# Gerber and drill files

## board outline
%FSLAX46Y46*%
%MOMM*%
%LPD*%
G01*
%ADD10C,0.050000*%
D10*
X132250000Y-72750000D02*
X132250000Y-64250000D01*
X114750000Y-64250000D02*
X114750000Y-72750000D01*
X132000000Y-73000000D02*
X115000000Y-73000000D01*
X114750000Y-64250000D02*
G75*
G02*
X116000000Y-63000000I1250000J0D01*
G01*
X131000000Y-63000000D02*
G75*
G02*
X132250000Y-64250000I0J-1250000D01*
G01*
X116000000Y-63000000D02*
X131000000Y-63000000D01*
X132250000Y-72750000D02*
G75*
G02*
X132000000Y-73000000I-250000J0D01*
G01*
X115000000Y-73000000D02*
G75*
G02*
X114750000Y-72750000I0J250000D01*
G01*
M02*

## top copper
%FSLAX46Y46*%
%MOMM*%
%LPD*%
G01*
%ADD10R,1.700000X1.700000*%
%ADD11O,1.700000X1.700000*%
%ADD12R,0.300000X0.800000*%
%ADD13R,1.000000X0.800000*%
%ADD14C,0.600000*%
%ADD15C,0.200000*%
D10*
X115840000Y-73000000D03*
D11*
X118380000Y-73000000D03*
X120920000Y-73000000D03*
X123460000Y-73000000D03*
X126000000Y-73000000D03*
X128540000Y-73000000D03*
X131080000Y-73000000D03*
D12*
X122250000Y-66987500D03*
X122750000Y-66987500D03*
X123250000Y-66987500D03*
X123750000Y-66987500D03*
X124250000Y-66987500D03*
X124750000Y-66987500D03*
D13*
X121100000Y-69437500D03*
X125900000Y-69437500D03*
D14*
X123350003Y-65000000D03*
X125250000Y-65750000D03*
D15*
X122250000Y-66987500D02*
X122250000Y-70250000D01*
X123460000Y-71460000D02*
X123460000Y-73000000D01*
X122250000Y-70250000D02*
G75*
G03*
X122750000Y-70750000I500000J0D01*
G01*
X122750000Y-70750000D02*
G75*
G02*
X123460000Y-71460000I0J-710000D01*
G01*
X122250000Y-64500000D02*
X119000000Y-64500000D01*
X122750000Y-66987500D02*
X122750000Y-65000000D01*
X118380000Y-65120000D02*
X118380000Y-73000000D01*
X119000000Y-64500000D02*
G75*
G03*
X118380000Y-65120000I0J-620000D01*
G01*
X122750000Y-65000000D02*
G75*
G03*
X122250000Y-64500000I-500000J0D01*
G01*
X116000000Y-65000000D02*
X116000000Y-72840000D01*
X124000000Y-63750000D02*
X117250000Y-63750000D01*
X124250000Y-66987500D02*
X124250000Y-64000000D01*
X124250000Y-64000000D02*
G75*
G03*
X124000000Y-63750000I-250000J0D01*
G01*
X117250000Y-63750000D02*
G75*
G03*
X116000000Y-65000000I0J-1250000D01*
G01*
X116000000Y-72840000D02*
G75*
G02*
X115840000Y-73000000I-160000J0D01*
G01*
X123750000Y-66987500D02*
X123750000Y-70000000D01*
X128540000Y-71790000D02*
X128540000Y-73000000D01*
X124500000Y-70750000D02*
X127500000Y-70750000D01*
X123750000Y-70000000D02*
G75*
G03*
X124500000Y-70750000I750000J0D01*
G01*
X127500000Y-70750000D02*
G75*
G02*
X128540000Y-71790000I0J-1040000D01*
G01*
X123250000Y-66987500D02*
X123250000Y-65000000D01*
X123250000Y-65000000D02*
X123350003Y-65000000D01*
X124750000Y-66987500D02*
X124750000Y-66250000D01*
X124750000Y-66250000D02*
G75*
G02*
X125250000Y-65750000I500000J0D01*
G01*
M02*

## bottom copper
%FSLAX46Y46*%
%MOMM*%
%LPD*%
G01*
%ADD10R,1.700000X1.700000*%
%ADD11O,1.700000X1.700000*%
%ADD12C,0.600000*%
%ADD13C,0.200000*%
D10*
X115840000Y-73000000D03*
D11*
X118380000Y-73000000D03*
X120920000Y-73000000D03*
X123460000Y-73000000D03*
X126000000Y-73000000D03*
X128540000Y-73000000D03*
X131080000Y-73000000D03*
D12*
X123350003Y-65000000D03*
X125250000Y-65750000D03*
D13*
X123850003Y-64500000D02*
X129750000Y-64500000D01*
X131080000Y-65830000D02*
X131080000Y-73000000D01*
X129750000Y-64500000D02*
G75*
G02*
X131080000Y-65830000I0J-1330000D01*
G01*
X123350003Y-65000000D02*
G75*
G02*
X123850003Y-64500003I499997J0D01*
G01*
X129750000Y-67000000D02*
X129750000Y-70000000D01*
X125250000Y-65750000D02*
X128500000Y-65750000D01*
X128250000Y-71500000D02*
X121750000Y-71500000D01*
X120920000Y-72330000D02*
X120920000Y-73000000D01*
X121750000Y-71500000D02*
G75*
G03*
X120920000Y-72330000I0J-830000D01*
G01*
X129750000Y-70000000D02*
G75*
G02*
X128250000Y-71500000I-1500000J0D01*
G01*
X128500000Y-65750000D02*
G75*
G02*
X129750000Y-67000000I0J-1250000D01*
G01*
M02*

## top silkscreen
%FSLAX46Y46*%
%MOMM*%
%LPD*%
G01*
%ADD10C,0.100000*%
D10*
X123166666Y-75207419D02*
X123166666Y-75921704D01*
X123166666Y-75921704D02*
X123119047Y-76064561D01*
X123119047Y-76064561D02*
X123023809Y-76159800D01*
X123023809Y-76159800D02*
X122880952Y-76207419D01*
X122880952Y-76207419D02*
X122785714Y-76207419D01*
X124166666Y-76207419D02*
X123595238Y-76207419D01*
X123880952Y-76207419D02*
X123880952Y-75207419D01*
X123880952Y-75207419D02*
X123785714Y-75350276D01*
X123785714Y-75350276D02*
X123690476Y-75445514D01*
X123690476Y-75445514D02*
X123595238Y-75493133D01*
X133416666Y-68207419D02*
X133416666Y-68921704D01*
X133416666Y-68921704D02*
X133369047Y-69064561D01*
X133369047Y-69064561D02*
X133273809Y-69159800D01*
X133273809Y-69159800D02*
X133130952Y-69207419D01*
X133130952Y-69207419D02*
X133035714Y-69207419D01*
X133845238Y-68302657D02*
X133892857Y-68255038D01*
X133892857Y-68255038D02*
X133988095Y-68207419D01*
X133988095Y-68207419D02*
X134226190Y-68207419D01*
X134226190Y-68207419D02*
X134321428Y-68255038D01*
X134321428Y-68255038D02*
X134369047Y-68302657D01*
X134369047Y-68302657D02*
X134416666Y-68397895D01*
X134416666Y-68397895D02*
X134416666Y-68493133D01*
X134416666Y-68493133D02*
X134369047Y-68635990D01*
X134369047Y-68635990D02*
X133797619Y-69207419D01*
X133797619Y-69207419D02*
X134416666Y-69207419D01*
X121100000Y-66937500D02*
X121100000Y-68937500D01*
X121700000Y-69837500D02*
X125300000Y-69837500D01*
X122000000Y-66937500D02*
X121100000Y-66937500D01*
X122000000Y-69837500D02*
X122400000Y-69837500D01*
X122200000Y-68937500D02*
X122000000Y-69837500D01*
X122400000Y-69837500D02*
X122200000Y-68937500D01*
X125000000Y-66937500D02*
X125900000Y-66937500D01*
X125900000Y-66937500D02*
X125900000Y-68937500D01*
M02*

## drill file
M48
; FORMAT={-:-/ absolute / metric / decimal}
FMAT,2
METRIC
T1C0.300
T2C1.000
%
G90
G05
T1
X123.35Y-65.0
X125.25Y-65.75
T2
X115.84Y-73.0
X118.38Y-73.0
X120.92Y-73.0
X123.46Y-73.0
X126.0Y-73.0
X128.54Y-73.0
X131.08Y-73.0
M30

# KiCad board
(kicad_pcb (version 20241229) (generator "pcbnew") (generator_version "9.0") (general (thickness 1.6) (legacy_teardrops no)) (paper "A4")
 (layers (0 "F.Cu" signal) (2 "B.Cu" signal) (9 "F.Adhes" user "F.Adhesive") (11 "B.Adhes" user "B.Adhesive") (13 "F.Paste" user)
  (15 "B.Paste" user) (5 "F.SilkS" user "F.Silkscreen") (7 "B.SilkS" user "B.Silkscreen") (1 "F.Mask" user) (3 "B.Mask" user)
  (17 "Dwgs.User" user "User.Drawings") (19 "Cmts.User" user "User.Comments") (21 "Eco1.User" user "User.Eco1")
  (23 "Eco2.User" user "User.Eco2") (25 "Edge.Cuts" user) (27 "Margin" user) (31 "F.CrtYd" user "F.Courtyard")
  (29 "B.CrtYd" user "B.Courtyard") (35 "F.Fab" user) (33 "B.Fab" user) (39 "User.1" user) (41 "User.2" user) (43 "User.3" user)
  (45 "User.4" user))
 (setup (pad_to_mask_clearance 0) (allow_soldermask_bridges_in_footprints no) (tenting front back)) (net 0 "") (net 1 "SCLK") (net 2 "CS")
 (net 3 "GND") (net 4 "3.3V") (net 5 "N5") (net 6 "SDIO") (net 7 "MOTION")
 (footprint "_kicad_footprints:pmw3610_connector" (layer "F.Cu") (at 123.46 73 90)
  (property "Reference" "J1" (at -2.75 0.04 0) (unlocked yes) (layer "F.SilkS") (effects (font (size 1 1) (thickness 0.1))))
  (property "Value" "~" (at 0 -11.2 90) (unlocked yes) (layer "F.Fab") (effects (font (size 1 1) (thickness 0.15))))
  (pad "1" thru_hole rect (at 0 -7.62 90) (size 1.7 1.7) (drill 1) (layers "*.Cu" "*.Mask") (remove_unused_layers no) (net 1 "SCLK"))
  (pad "2" thru_hole oval (at 0 -5.08 90) (size 1.7 1.7) (drill 1) (layers "*.Cu" "*.Mask") (remove_unused_layers no) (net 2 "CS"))
  (pad "3" thru_hole oval (at 0 -2.54 90) (size 1.7 1.7) (drill 1) (layers "*.Cu" "*.Mask") (remove_unused_layers no) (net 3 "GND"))
  (pad "4" thru_hole oval (at 0 0 90) (size 1.7 1.7) (drill 1) (layers "*.Cu" "*.Mask") (remove_unused_layers no) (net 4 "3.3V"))
  (pad "5" thru_hole oval (at 0 2.54 90) (size 1.7 1.7) (drill 1) (layers "*.Cu" "*.Mask") (remove_unused_layers no) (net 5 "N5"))
  (pad "6" thru_hole oval (at 0 5.08 90) (size 1.7 1.7) (drill 1) (layers "*.Cu" "*.Mask") (remove_unused_layers no) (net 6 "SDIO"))
  (pad "7" thru_hole oval (at 0 7.62 90) (size 1.7 1.7) (drill 1) (layers "*.Cu" "*.Mask") (remove_unused_layers no) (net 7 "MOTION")))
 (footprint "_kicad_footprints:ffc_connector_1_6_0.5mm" (layer "F.Cu") (at 123.5 75.2375)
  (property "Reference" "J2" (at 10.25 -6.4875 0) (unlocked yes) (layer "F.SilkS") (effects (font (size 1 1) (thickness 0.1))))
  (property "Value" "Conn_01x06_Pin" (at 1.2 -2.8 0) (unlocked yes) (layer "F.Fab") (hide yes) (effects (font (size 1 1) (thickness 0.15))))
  (fp_line (start -2.4 -8.3) (end -2.4 -6.3) (stroke (width 0.1) (type default)) (layer "F.SilkS"))
  (fp_line (start -1.8 -5.4) (end 1.8 -5.4) (stroke (width 0.1) (type default)) (layer "F.SilkS"))
  (fp_line (start -1.5 -8.3) (end -2.4 -8.3) (stroke (width 0.1) (type default)) (layer "F.SilkS"))
  (fp_line (start -1.5 -5.4) (end -1.1 -5.4) (stroke (width 0.1) (type default)) (layer "F.SilkS"))
  (fp_line (start -1.3 -6.3) (end -1.5 -5.4) (stroke (width 0.1) (type default)) (layer "F.SilkS"))
  (fp_line (start -1.1 -5.4) (end -1.3 -6.3) (stroke (width 0.1) (type default)) (layer "F.SilkS"))
  (fp_line (start 1.5 -8.3) (end 2.4 -8.3) (stroke (width 0.1) (type default)) (layer "F.SilkS"))
  (fp_line (start 2.4 -8.3) (end 2.4 -6.3) (stroke (width 0.1) (type default)) (layer "F.SilkS"))
  (pad "1" smd rect (at -1.25 -8.25) (size 0.3 0.8) (layers "F.Cu" "F.Mask" "F.Paste") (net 4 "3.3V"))
  (pad "2" smd rect (at -0.75 -8.25) (size 0.3 0.8) (layers "F.Cu" "F.Mask" "F.Paste") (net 2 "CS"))
  (pad "3" smd rect (at -0.25 -8.25) (size 0.3 0.8) (layers "F.Cu" "F.Mask" "F.Paste") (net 7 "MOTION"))
  (pad "4" smd rect (at 0.25 -8.25) (size 0.3 0.8) (layers "F.Cu" "F.Mask" "F.Paste") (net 6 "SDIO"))
  (pad "5" smd rect (at 0.75 -8.25) (size 0.3 0.8) (layers "F.Cu" "F.Mask" "F.Paste") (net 1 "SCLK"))
  (pad "6" smd rect (at 1.25 -8.25) (size 0.3 0.8) (layers "F.Cu" "F.Mask" "F.Paste") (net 3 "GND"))
  (pad "MP" smd rect (at -2.4 -5.8) (size 1 0.8) (layers "F.Cu" "F.Mask" "F.Paste"))
  (pad "MP" smd rect (at 2.4 -5.8) (size 1 0.8) (layers "F.Cu" "F.Mask" "F.Paste")))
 (gr_line (start 132.25 72.75) (end 132.25 64.25) (stroke (width 0.05) (type default)) (layer "Edge.Cuts"))
 (gr_line (start 114.75 64.25) (end 114.75 72.75) (stroke (width 0.05) (type default)) (layer "Edge.Cuts"))
 (gr_line (start 132 73) (end 115 73) (stroke (width 0.05) (type default)) (layer "Edge.Cuts"))
 (gr_arc (start 114.75 64.25) (mid 115.116117 63.366117) (end 116 63) (stroke (width 0.05) (type default)) (layer "Edge.Cuts"))
 (gr_arc (start 131 63) (mid 131.883883 63.366117) (end 132.25 64.25) (stroke (width 0.05) (type default)) (layer "Edge.Cuts"))
 (gr_line (start 116 63) (end 131 63) (stroke (width 0.05) (type default)) (layer "Edge.Cuts"))
 (gr_arc (start 132.25 72.75) (mid 132.176777 72.926777) (end 132 73) (stroke (width 0.05) (type default)) (layer "Edge.Cuts"))
 (gr_arc (start 115 73) (mid 114.823223 72.926777) (end 114.75 72.75) (stroke (width 0.05) (type default)) (layer "Edge.Cuts"))
 (segment (start 122.25 66.9875) (end 122.25 70.25) (width 0.2) (layer "F.Cu") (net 4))
 (segment (start 123.46 71.46) (end 123.46 73) (width 0.2) (layer "F.Cu") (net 4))
 (arc (start 122.25 70.25) (mid 122.396447 70.603553) (end 122.75 70.75) (width 0.2) (layer "F.Cu") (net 4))
 (arc (start 122.75 70.75) (mid 123.252046 70.957954) (end 123.46 71.46) (width 0.2) (layer "F.Cu") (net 4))
 (segment (start 122.25 64.5) (end 119 64.5) (width 0.2) (layer "F.Cu") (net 2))
 (segment (start 122.75 66.9875) (end 122.75 65) (width 0.2) (layer "F.Cu") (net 2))
 (segment (start 118.38 65.12) (end 118.38 73) (width 0.2) (layer "F.Cu") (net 2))
 (arc (start 119 64.5) (mid 118.561594 64.681594) (end 118.38 65.12) (width 0.2) (layer "F.Cu") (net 2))
 (arc (start 122.75 65) (mid 122.603553 64.646447) (end 122.25 64.5) (width 0.2) (layer "F.Cu") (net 2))
 (segment (start 116 65) (end 116 72.84) (width 0.2) (layer "F.Cu") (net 1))
 (segment (start 124 63.75) (end 117.25 63.75) (width 0.2) (layer "F.Cu") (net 1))
 (segment (start 124.25 66.9875) (end 124.25 64) (width 0.2) (layer "F.Cu") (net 1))
 (arc (start 124.25 64) (mid 124.176777 63.823223) (end 124 63.75) (width 0.2) (layer "F.Cu") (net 1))
 (arc (start 117.25 63.75) (mid 116.366117 64.116117) (end 116 65) (width 0.2) (layer "F.Cu") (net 1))
 (arc (start 116 72.84) (mid 115.953137 72.953137) (end 115.84 73) (width 0.2) (layer "F.Cu") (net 1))
 (segment (start 123.75 66.9875) (end 123.75 70) (width 0.2) (layer "F.Cu") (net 6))
 (segment (start 128.54 71.79) (end 128.54 73) (width 0.2) (layer "F.Cu") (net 6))
 (segment (start 124.5 70.75) (end 127.5 70.75) (width 0.2) (layer "F.Cu") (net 6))
 (arc (start 123.75 70) (mid 123.96967 70.53033) (end 124.5 70.75) (width 0.2) (layer "F.Cu") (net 6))
 (arc (start 127.5 70.75) (mid 128.235391 71.054609) (end 128.54 71.79) (width 0.2) (layer "F.Cu") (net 6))
 (segment (start 123.25 66.9875) (end 123.25 65) (width 0.2) (layer "F.Cu") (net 7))
 (segment (start 123.25 65) (end 123.350003 65) (width 0.2) (layer "F.Cu") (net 7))
 (via (at 123.350003 65) (size 0.6) (drill 0.3) (layers "F.Cu" "B.Cu") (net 7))
 (segment (start 123.850003 64.5) (end 129.75 64.5) (width 0.2) (layer "B.Cu") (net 7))
 (segment (start 131.08 65.83) (end 131.08 73) (width 0.2) (layer "B.Cu") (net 7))
 (arc (start 129.75 64.5) (mid 130.690452 64.889548) (end 131.08 65.83) (width 0.2) (layer "B.Cu") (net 7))
 (arc (start 123.350003 65) (mid 123.49645 64.646447) (end 123.850003 64.5) (width 0.2) (layer "B.Cu") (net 7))
 (segment (start 124.75 66.9875) (end 124.75 66.25) (width 0.2) (layer "F.Cu") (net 3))
 (via (at 125.25 65.75) (size 0.6) (drill 0.3) (layers "F.Cu" "B.Cu") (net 3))
 (arc (start 124.75 66.25) (mid 124.896447 65.896447) (end 125.25 65.75) (width 0.2) (layer "F.Cu") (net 3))
 (segment (start 129.75 67) (end 129.75 70) (width 0.2) (layer "B.Cu") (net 3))
 (segment (start 125.25 65.75) (end 128.5 65.75) (width 0.2) (layer "B.Cu") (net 3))
 (segment (start 128.25 71.5) (end 121.75 71.5) (width 0.2) (layer "B.Cu") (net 3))
 (segment (start 120.92 72.33) (end 120.92 73) (width 0.2) (layer "B.Cu") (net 3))
 (arc (start 121.75 71.5) (mid 121.163101 71.743101) (end 120.92 72.33) (width 0.2) (layer "B.Cu") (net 3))
 (arc (start 129.75 70) (mid 129.31066 71.06066) (end 128.25 71.5) (width 0.2) (layer "B.Cu") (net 3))
 (arc (start 128.5 65.75) (mid 129.383883 66.116117) (end 129.75 67) (width 0.2) (layer "B.Cu") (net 3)))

